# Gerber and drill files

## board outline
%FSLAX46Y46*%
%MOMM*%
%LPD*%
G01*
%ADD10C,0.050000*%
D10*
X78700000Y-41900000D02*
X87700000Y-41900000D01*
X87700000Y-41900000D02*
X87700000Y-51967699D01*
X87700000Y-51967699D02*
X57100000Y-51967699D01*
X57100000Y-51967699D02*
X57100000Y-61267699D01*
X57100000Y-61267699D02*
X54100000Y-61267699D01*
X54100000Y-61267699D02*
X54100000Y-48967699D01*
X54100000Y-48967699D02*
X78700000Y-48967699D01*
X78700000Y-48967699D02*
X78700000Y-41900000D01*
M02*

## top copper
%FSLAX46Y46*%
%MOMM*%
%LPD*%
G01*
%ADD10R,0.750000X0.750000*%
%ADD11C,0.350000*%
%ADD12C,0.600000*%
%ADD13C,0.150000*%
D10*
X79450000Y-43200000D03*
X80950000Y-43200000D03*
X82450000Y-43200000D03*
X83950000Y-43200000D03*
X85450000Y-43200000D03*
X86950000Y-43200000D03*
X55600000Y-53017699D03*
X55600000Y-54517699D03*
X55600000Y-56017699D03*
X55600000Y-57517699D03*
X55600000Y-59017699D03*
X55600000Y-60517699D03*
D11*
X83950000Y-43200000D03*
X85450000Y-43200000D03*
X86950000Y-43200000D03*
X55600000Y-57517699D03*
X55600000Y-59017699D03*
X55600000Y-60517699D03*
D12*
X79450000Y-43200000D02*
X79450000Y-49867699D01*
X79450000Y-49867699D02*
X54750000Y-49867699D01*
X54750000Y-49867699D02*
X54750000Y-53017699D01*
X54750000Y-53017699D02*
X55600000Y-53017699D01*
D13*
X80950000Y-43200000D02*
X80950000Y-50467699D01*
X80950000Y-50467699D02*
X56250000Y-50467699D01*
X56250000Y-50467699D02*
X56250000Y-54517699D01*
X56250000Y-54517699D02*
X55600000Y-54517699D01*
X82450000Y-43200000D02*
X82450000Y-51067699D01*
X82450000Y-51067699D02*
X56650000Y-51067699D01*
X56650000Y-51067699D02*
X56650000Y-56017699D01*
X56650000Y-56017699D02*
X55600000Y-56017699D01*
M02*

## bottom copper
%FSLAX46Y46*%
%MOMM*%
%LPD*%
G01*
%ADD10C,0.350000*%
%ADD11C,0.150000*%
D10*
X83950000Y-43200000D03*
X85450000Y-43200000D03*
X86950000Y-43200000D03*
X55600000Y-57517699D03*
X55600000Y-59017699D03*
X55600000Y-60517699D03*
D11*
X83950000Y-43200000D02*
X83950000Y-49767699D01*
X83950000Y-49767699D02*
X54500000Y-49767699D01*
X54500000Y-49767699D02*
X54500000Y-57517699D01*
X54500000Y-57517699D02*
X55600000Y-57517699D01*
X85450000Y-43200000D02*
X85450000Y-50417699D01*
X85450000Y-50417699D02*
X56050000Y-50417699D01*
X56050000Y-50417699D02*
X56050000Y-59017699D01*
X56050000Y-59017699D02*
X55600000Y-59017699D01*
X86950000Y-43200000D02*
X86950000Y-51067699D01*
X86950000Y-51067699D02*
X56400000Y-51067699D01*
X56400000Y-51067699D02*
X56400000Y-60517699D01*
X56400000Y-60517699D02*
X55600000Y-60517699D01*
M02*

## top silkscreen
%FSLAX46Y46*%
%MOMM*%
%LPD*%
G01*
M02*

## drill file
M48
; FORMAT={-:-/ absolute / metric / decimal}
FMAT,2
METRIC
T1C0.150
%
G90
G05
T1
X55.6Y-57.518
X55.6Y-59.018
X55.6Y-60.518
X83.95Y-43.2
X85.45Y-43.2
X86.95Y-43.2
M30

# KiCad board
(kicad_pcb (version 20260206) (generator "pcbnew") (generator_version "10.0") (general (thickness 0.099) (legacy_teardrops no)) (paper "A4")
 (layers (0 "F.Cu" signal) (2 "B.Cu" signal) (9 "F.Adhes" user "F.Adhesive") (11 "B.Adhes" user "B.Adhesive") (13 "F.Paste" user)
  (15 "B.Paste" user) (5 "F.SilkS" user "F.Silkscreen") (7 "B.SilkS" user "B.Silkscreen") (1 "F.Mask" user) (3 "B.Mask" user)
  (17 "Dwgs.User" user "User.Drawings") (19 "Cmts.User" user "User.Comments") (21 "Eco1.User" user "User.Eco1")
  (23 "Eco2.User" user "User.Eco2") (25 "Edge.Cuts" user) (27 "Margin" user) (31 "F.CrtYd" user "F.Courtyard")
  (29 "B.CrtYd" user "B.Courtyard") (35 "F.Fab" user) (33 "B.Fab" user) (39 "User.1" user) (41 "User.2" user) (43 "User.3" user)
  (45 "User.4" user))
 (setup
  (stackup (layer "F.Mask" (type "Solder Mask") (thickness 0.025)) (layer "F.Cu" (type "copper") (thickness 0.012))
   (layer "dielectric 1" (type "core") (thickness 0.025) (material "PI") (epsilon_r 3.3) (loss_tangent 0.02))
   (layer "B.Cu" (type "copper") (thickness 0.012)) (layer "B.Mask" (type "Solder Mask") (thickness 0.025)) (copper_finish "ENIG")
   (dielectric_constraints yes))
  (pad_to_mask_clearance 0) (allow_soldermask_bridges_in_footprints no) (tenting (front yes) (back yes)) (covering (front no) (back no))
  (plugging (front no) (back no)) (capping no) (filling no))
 (gr_line (start 78.7 41.90000000000001) (end 87.7 41.90000000000001) (stroke (width 0.05) (type default)) (layer "Edge.Cuts"))
 (gr_line (start 87.7 41.90000000000001) (end 87.7 51.96769878025519) (stroke (width 0.05) (type default)) (layer "Edge.Cuts"))
 (gr_line (start 87.7 51.96769878025519) (end 57.1 51.96769878025519) (stroke (width 0.05) (type default)) (layer "Edge.Cuts"))
 (gr_line (start 57.1 51.96769878025519) (end 57.1 61.26769878025519) (stroke (width 0.05) (type default)) (layer "Edge.Cuts"))
 (gr_line (start 57.1 61.26769878025519) (end 54.1 61.26769878025519) (stroke (width 0.05) (type default)) (layer "Edge.Cuts"))
 (gr_line (start 54.1 61.26769878025519) (end 54.1 48.96769878025519) (stroke (width 0.05) (type default)) (layer "Edge.Cuts"))
 (gr_line (start 54.1 48.96769878025519) (end 78.7 48.96769878025519) (stroke (width 0.05) (type default)) (layer "Edge.Cuts"))
 (gr_line (start 78.7 48.96769878025519) (end 78.7 41.90000000000001) (stroke (width 0.05) (type default)) (layer "Edge.Cuts"))
 (via (at 83.95 43.2) (size 0.35) (drill 0.15) (layers "F.Cu" "B.Cu") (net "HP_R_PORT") (locked yes))
 (via (at 85.45 43.2) (size 0.35) (drill 0.15) (layers "F.Cu" "B.Cu") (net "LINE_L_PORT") (locked yes))
 (via (at 86.95 43.2) (size 0.35) (drill 0.15) (layers "F.Cu" "B.Cu") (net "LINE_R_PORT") (locked yes))
 (via (at 55.599999999999994 57.51769878025519) (size 0.35) (drill 0.15) (layers "F.Cu" "B.Cu") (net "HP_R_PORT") (locked yes))
 (via (at 55.599999999999994 59.01769878025519) (size 0.35) (drill 0.15) (layers "F.Cu" "B.Cu") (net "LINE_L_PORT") (locked yes))
 (via (at 55.599999999999994 60.51769878025519) (size 0.35) (drill 0.15) (layers "F.Cu" "B.Cu") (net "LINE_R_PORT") (locked yes))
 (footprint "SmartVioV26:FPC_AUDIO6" (layer "F.Cu") (at 0 0)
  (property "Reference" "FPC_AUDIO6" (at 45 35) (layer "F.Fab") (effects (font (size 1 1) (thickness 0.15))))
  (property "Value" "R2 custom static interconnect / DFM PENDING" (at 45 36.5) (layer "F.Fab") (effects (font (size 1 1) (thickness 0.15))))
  (pad "S1" smd rect (at 79.45 43.2) (size 0.75 0.75) (layers "F.Cu" "F.Mask") (solder_mask_margin 0.1) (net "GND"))
  (pad "S2" smd rect (at 80.95 43.2) (size 0.75 0.75) (layers "F.Cu" "F.Mask") (solder_mask_margin 0.1) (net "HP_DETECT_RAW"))
  (pad "S3" smd rect (at 82.45 43.2) (size 0.75 0.75) (layers "F.Cu" "F.Mask") (solder_mask_margin 0.1) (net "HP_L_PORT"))
  (pad "S4" smd rect (at 83.95 43.2) (size 0.75 0.75) (layers "F.Cu" "F.Mask") (solder_mask_margin 0.1) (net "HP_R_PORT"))
  (pad "S5" smd rect (at 85.45 43.2) (size 0.75 0.75) (layers "F.Cu" "F.Mask") (solder_mask_margin 0.1) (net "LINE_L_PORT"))
  (pad "S6" smd rect (at 86.95 43.2) (size 0.75 0.75) (layers "F.Cu" "F.Mask") (solder_mask_margin 0.1) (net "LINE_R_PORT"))
  (pad "T1" smd rect (at 55.599999999999994 53.01769878025519) (size 0.75 0.75) (layers "F.Cu" "F.Mask") (solder_mask_margin 0.1)
   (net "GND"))
  (pad "T2" smd rect (at 55.599999999999994 54.51769878025519) (size 0.75 0.75) (layers "F.Cu" "F.Mask") (solder_mask_margin 0.1)
   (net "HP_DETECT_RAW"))
  (pad "T3" smd rect (at 55.599999999999994 56.01769878025519) (size 0.75 0.75) (layers "F.Cu" "F.Mask") (solder_mask_margin 0.1)
   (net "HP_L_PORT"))
  (pad "T4" smd rect (at 55.599999999999994 57.51769878025519) (size 0.75 0.75) (layers "F.Cu" "F.Mask") (solder_mask_margin 0.1)
   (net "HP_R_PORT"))
  (pad "T5" smd rect (at 55.599999999999994 59.01769878025519) (size 0.75 0.75) (layers "F.Cu" "F.Mask") (solder_mask_margin 0.1)
   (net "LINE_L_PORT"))
  (pad "T6" smd rect (at 55.599999999999994 60.51769878025519) (size 0.75 0.75) (layers "F.Cu" "F.Mask") (solder_mask_margin 0.1)
   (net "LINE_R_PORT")))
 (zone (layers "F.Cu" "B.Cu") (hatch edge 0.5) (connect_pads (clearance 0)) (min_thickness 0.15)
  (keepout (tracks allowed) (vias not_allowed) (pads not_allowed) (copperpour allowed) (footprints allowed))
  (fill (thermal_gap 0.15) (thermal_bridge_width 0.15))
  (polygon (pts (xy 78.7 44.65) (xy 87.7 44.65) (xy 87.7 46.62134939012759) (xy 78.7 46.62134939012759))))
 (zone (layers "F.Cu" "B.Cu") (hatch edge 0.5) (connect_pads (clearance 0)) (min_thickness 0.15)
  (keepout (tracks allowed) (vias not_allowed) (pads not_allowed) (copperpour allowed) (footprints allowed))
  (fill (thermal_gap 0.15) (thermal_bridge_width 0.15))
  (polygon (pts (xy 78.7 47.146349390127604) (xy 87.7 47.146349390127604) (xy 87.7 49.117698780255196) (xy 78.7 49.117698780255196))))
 (segment (start 79.45 43.2) (end 79.45 49.867698780255196) (width 0.6) (layer "F.Cu") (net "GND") (locked yes))
 (segment (start 79.45 49.867698780255196) (end 54.75 49.867698780255196) (width 0.6) (layer "F.Cu") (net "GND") (locked yes))
 (segment (start 54.75 49.867698780255196) (end 54.75 53.01769878025519) (width 0.6) (layer "F.Cu") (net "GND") (locked yes))
 (segment (start 54.75 53.01769878025519) (end 55.599999999999994 53.01769878025519) (width 0.6) (layer "F.Cu") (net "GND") (locked yes))
 (segment (start 80.95 43.2) (end 80.95 50.4676987802552) (width 0.15) (layer "F.Cu") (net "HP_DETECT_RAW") (locked yes))
 (segment (start 80.95 50.4676987802552) (end 56.25 50.4676987802552) (width 0.15) (layer "F.Cu") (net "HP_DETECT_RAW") (locked yes))
 (segment (start 56.25 50.4676987802552) (end 56.25 54.51769878025519) (width 0.15) (layer "F.Cu") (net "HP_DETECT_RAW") (locked yes))
 (segment (start 56.25 54.51769878025519) (end 55.599999999999994 54.51769878025519) (width 0.15) (layer "F.Cu") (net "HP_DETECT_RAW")
  (locked yes))
 (segment (start 82.45 43.2) (end 82.45 51.0676987802552) (width 0.15) (layer "F.Cu") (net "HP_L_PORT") (locked yes))
 (segment (start 82.45 51.0676987802552) (end 56.65 51.0676987802552) (width 0.15) (layer "F.Cu") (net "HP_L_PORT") (locked yes))
 (segment (start 56.65 51.0676987802552) (end 56.65 56.01769878025519) (width 0.15) (layer "F.Cu") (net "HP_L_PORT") (locked yes))
 (segment (start 56.65 56.01769878025519) (end 55.599999999999994 56.01769878025519) (width 0.15) (layer "F.Cu") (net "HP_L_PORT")
  (locked yes))
 (segment (start 83.95 43.2) (end 83.95 49.767698780255195) (width 0.15) (layer "B.Cu") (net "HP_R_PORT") (locked yes))
 (segment (start 83.95 49.767698780255195) (end 54.5 49.767698780255195) (width 0.15) (layer "B.Cu") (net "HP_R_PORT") (locked yes))
 (segment (start 54.5 49.767698780255195) (end 54.5 57.51769878025519) (width 0.15) (layer "B.Cu") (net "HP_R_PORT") (locked yes))
 (segment (start 54.5 57.51769878025519) (end 55.599999999999994 57.51769878025519) (width 0.15) (layer "B.Cu") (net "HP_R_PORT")
  (locked yes))
 (segment (start 85.45 43.2) (end 85.45 50.41769878025519) (width 0.15) (layer "B.Cu") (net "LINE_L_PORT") (locked yes))
 (segment (start 85.45 50.41769878025519) (end 56.05 50.41769878025519) (width 0.15) (layer "B.Cu") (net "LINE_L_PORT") (locked yes))
 (segment (start 56.05 50.41769878025519) (end 56.05 59.01769878025519) (width 0.15) (layer "B.Cu") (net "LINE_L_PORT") (locked yes))
 (segment (start 56.05 59.01769878025519) (end 55.599999999999994 59.01769878025519) (width 0.15) (layer "B.Cu") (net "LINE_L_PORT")
  (locked yes))
 (segment (start 86.95 43.2) (end 86.95 51.0676987802552) (width 0.15) (layer "B.Cu") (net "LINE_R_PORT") (locked yes))
 (segment (start 86.95 51.0676987802552) (end 56.4 51.0676987802552) (width 0.15) (layer "B.Cu") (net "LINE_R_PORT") (locked yes))
 (segment (start 56.4 51.0676987802552) (end 56.4 60.51769878025519) (width 0.15) (layer "B.Cu") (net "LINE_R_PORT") (locked yes))
 (segment (start 56.4 60.51769878025519) (end 55.599999999999994 60.51769878025519) (width 0.15) (layer "B.Cu") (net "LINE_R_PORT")
  (locked yes)))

